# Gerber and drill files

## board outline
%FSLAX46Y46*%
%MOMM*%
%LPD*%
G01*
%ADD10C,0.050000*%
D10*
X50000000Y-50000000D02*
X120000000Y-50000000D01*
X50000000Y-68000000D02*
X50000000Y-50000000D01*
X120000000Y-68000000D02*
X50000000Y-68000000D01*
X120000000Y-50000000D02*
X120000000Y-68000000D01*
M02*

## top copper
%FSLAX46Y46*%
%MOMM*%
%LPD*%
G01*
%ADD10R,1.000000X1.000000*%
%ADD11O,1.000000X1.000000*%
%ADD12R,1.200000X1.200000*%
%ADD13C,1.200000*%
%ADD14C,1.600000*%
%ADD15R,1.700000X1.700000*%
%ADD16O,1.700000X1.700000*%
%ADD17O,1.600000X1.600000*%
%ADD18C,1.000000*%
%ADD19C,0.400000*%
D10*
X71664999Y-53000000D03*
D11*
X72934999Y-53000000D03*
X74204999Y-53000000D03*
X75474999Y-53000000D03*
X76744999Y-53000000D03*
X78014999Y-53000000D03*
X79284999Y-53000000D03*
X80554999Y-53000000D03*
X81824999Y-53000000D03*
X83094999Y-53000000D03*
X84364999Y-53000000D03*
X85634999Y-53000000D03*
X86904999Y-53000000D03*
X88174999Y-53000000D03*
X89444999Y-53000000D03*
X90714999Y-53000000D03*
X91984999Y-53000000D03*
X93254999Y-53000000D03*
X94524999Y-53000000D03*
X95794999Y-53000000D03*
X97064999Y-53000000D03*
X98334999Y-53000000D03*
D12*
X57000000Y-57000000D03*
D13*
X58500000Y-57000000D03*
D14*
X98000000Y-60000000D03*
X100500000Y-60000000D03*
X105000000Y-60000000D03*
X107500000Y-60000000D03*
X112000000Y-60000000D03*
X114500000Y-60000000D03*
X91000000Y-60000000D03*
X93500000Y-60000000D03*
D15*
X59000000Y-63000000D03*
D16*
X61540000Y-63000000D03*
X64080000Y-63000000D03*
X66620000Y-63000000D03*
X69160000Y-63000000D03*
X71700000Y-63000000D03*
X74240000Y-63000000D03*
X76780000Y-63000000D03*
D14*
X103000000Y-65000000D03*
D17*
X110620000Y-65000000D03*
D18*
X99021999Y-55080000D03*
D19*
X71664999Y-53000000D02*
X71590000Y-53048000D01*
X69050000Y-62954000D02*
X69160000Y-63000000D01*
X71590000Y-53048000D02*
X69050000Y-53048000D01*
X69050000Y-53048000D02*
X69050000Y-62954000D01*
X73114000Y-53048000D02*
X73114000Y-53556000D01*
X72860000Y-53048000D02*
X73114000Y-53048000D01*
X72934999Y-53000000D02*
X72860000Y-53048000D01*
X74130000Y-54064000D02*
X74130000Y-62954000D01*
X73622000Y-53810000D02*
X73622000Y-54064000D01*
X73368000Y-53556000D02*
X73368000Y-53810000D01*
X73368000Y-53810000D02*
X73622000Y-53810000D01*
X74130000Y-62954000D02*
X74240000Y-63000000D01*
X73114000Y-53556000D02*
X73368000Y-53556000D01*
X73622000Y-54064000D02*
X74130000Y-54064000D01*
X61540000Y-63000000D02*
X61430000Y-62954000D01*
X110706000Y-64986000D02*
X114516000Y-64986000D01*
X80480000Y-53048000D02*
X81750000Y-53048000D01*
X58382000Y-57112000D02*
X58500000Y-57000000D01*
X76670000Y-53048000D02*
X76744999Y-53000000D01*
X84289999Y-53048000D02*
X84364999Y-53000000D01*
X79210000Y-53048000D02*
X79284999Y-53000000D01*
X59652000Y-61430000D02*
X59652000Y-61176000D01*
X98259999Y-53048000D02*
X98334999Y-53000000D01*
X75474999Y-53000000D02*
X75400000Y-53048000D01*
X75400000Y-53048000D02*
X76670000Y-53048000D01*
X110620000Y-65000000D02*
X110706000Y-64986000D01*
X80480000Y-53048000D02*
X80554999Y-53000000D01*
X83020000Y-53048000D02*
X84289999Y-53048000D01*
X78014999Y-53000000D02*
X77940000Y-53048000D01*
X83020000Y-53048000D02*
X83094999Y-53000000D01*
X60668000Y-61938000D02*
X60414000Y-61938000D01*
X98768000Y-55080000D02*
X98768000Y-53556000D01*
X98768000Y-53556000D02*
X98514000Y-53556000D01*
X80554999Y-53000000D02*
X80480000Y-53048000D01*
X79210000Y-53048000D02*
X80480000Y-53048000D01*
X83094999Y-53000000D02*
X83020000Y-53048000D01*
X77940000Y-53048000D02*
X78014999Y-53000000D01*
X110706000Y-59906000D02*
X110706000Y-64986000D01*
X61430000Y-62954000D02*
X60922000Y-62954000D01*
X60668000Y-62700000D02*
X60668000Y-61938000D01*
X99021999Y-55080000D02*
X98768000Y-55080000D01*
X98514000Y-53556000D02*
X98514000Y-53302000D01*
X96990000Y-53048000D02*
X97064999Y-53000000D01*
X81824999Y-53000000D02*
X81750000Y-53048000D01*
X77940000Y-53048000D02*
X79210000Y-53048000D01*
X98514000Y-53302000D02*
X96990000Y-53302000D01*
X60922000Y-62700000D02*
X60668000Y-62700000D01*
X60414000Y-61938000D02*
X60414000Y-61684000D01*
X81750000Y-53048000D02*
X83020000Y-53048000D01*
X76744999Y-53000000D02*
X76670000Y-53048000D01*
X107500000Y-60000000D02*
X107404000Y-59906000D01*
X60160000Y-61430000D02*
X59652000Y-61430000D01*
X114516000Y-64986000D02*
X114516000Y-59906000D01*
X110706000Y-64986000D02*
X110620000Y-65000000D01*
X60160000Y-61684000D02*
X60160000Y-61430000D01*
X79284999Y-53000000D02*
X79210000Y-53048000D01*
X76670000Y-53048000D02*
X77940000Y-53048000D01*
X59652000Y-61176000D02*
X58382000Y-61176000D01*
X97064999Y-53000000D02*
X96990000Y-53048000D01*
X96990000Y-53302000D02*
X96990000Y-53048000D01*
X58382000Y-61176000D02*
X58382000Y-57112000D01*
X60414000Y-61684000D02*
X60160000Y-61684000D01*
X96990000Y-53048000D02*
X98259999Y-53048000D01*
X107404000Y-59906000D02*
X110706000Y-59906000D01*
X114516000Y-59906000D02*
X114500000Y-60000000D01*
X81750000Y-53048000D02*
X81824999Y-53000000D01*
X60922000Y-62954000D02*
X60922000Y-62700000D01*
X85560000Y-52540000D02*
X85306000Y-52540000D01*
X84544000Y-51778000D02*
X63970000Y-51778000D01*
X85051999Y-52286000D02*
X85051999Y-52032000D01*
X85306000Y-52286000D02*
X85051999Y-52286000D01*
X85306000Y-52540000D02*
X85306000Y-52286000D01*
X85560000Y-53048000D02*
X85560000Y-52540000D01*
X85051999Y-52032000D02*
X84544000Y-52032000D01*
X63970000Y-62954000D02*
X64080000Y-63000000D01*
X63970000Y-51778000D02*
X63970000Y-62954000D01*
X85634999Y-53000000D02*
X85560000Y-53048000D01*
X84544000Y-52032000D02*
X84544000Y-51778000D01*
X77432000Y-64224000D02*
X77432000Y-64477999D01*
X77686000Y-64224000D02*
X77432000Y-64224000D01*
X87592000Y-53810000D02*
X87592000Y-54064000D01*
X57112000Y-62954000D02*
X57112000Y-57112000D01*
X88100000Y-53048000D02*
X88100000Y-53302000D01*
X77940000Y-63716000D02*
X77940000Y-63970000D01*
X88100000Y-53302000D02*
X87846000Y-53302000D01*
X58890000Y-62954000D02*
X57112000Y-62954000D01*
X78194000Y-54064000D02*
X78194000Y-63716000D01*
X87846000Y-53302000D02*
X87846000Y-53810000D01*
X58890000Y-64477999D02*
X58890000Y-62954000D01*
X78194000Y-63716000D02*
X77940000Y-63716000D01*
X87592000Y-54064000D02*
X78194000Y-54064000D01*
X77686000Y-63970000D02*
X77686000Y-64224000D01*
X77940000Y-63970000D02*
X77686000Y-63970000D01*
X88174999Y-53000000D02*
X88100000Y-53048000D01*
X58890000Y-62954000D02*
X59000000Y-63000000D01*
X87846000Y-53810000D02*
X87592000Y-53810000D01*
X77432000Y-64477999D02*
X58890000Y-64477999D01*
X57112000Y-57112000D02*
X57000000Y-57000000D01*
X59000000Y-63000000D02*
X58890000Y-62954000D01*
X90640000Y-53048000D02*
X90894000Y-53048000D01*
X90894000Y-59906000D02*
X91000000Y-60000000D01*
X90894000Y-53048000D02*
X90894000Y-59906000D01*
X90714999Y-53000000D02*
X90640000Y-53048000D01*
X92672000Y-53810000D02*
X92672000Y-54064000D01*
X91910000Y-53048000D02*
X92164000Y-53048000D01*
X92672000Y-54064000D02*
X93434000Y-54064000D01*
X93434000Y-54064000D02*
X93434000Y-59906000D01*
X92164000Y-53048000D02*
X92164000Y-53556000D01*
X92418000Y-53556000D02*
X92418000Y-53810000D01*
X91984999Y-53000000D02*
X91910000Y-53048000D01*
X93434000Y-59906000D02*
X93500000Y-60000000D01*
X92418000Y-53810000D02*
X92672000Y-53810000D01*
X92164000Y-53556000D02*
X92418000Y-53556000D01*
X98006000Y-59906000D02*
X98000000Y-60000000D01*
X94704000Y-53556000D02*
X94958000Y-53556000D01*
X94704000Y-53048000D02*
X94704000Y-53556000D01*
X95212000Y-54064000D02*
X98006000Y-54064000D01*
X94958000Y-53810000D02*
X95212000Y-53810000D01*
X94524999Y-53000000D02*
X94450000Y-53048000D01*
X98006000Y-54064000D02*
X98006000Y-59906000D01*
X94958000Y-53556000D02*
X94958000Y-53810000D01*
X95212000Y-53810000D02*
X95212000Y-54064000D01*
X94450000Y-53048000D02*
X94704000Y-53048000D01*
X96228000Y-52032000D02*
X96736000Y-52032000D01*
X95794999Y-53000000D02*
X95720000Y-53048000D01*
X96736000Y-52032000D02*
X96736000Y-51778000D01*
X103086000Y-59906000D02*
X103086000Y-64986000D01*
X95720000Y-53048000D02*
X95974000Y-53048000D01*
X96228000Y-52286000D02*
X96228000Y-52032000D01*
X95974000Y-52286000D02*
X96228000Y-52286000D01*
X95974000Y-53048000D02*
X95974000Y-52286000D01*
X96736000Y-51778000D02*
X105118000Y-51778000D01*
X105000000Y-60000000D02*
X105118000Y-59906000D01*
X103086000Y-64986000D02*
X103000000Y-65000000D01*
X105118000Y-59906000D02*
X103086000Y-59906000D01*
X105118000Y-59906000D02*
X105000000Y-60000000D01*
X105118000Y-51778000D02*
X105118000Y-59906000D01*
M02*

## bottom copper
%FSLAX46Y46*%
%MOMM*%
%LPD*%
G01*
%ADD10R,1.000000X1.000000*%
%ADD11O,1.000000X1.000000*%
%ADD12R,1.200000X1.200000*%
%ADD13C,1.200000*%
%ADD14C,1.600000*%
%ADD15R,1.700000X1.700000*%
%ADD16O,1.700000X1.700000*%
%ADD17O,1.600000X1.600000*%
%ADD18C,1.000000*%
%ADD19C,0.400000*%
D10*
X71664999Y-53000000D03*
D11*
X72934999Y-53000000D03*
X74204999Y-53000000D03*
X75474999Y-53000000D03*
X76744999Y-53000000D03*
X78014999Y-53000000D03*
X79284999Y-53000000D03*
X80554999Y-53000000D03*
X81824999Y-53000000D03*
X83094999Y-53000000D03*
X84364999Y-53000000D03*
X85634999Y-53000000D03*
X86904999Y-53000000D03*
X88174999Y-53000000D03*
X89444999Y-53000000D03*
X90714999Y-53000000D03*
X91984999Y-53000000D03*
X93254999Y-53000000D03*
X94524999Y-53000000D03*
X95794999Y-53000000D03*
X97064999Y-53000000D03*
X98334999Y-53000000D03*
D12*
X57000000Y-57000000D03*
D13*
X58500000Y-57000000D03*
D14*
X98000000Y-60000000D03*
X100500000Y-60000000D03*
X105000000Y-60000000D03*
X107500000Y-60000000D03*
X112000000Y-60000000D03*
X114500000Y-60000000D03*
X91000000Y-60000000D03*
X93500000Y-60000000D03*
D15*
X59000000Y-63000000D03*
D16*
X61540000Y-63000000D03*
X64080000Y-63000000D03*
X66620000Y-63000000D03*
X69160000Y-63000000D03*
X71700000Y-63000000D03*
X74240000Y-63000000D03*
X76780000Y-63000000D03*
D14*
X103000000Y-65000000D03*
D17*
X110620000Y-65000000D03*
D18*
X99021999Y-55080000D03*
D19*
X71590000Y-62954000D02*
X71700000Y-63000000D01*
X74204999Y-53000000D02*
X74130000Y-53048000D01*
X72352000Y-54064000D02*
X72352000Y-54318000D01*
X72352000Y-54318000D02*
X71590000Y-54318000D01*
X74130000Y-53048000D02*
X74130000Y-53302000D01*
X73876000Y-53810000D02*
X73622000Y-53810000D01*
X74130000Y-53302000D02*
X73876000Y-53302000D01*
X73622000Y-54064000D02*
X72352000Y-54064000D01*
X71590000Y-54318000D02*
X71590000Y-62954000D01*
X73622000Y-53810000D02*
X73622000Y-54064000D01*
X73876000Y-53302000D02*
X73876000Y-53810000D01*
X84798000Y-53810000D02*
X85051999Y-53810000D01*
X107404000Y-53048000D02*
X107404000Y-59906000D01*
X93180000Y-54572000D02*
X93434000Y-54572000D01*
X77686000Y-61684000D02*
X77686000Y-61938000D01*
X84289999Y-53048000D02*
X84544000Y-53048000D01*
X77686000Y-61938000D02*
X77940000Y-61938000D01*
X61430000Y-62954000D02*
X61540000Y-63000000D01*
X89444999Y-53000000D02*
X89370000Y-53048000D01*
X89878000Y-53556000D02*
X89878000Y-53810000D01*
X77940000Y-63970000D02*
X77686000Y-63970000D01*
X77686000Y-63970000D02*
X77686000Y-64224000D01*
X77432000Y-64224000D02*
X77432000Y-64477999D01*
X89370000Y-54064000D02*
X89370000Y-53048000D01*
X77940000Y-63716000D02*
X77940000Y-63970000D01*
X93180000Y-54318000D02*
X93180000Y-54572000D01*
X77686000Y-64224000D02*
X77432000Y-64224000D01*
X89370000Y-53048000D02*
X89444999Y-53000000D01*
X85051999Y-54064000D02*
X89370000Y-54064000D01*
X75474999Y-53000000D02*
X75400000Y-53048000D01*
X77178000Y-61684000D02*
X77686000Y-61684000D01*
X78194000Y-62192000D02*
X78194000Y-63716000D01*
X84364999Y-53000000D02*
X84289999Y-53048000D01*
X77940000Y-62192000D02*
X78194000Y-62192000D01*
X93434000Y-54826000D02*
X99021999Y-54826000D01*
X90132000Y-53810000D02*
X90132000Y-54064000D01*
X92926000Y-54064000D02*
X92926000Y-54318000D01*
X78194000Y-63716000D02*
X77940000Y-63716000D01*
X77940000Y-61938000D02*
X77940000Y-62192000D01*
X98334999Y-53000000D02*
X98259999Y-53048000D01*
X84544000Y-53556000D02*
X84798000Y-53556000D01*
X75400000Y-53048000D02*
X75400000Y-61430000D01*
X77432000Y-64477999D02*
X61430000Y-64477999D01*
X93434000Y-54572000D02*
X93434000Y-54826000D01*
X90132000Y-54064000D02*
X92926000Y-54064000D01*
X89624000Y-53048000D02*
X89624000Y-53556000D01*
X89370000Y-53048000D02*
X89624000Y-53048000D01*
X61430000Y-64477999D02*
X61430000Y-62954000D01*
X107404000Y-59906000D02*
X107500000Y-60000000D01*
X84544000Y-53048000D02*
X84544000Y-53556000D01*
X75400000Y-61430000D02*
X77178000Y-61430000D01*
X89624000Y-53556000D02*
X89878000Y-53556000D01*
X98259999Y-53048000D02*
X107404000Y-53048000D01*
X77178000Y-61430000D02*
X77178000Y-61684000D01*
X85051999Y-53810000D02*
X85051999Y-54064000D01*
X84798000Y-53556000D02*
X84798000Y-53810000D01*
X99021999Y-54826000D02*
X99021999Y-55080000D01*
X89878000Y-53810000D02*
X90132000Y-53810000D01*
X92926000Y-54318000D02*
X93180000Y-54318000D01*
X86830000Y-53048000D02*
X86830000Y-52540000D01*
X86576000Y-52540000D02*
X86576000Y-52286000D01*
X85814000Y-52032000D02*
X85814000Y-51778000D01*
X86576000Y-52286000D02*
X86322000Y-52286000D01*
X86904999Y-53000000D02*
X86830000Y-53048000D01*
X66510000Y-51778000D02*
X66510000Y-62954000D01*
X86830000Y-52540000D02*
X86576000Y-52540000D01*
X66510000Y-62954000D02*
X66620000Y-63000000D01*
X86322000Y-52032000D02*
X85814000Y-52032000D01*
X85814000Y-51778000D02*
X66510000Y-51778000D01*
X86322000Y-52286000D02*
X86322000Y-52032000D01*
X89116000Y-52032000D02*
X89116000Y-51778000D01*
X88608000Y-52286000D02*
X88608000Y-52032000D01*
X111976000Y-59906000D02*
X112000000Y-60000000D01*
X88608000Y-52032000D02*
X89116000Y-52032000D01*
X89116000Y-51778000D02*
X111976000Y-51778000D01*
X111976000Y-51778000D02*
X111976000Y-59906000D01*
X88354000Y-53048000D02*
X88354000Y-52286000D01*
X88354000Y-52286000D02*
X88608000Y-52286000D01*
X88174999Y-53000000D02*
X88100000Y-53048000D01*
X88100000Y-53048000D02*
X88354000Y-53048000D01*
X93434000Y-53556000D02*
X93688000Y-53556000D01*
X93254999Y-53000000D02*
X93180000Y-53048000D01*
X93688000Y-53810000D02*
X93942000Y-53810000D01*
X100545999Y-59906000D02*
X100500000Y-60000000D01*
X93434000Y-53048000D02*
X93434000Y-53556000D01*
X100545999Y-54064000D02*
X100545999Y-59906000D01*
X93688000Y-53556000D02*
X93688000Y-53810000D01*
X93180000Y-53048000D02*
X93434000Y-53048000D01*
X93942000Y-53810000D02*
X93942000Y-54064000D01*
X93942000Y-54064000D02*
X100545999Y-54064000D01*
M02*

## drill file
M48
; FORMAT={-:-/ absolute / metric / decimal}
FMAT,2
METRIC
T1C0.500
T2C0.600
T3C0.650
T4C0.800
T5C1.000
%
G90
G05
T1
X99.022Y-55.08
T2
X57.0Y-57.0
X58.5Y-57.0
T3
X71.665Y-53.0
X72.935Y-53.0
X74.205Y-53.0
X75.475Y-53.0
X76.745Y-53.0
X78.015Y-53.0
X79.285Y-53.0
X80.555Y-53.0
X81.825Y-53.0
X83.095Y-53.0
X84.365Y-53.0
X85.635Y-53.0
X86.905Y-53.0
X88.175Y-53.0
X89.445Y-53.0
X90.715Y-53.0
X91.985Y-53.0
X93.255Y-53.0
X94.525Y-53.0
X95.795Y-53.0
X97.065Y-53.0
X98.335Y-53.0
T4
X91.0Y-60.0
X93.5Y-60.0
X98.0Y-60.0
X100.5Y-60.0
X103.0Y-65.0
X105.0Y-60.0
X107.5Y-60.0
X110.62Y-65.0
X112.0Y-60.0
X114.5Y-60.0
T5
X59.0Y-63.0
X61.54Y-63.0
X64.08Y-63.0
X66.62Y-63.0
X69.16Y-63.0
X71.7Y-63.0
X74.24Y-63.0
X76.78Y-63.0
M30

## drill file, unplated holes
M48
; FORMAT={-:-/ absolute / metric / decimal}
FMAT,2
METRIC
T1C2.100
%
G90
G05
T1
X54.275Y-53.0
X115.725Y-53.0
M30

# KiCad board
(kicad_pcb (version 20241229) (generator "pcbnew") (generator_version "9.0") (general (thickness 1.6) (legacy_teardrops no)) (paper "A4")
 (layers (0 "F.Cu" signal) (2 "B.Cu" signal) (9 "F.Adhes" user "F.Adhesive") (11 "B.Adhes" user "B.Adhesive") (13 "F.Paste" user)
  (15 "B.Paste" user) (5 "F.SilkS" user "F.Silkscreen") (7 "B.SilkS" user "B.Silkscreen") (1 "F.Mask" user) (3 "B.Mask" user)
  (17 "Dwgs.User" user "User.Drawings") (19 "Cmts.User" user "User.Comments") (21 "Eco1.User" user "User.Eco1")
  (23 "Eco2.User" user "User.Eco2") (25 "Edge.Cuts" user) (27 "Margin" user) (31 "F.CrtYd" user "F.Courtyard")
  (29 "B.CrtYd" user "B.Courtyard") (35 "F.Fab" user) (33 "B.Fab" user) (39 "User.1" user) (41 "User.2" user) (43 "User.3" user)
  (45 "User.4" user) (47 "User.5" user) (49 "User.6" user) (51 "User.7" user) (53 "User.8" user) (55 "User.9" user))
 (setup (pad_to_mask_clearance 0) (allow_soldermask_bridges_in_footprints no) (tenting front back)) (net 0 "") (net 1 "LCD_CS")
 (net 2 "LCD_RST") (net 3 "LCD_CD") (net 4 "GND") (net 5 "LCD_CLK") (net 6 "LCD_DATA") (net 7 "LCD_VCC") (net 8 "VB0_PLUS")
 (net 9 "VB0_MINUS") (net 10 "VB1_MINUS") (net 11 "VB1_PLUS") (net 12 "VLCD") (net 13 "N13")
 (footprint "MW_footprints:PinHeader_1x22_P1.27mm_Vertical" (layer "F.Cu") (at 71.664999 53 90)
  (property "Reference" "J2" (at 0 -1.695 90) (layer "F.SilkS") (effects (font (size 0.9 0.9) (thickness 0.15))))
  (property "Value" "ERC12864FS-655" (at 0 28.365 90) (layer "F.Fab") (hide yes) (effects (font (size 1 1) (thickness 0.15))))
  (pad "1" thru_hole rect (at 0 0 90) (size 1 1) (drill 0.65) (layers "*.Cu" "*.Mask") (remove_unused_layers no) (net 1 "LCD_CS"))
  (pad "2" thru_hole oval (at 0 1.27 90) (size 1 1) (drill 0.65) (layers "*.Cu" "*.Mask") (remove_unused_layers no) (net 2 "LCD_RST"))
  (pad "3" thru_hole oval (at 0 2.54 90) (size 1 1) (drill 0.65) (layers "*.Cu" "*.Mask") (remove_unused_layers no) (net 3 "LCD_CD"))
  (pad "4" thru_hole oval (at 0 3.81 90) (size 1 1) (drill 0.65) (layers "*.Cu" "*.Mask") (remove_unused_layers no) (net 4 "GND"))
  (pad "5" thru_hole oval (at 0 5.08 90) (size 1 1) (drill 0.65) (layers "*.Cu" "*.Mask") (remove_unused_layers no) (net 4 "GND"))
  (pad "6" thru_hole oval (at 0 6.35 90) (size 1 1) (drill 0.65) (layers "*.Cu" "*.Mask") (remove_unused_layers no) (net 4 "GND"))
  (pad "7" thru_hole oval (at 0 7.62 90) (size 1 1) (drill 0.65) (layers "*.Cu" "*.Mask") (remove_unused_layers no) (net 4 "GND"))
  (pad "8" thru_hole oval (at 0 8.89 90) (size 1 1) (drill 0.65) (layers "*.Cu" "*.Mask") (remove_unused_layers no) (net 4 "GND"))
  (pad "9" thru_hole oval (at 0 10.16 90) (size 1 1) (drill 0.65) (layers "*.Cu" "*.Mask") (remove_unused_layers no) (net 4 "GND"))
  (pad "10" thru_hole oval (at 0 11.43 90) (size 1 1) (drill 0.65) (layers "*.Cu" "*.Mask") (remove_unused_layers no) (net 4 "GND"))
  (pad "11" thru_hole oval (at 0 12.7 90) (size 1 1) (drill 0.65) (layers "*.Cu" "*.Mask") (remove_unused_layers no) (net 4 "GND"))
  (pad "12" thru_hole oval (at 0 13.97 90) (size 1 1) (drill 0.65) (layers "*.Cu" "*.Mask") (remove_unused_layers no) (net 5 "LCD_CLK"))
  (pad "13" thru_hole oval (at 0 15.24 90) (size 1 1) (drill 0.65) (layers "*.Cu" "*.Mask") (remove_unused_layers no) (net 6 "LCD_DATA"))
  (pad "14" thru_hole oval (at 0 16.51 90) (size 1 1) (drill 0.65) (layers "*.Cu" "*.Mask") (remove_unused_layers no) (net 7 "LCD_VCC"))
  (pad "15" thru_hole oval (at 0 17.78 90) (size 1 1) (drill 0.65) (layers "*.Cu" "*.Mask") (remove_unused_layers no) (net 4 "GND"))
  (pad "16" thru_hole oval (at 0 19.05 90) (size 1 1) (drill 0.65) (layers "*.Cu" "*.Mask") (remove_unused_layers no) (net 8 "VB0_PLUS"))
  (pad "17" thru_hole oval (at 0 20.32 90) (size 1 1) (drill 0.65) (layers "*.Cu" "*.Mask") (remove_unused_layers no) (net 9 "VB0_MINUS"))
  (pad "18" thru_hole oval (at 0 21.59 90) (size 1 1) (drill 0.65) (layers "*.Cu" "*.Mask") (remove_unused_layers no) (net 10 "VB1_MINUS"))
  (pad "19" thru_hole oval (at 0 22.86 90) (size 1 1) (drill 0.65) (layers "*.Cu" "*.Mask") (remove_unused_layers no) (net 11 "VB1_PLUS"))
  (pad "20" thru_hole oval (at 0 24.13 90) (size 1 1) (drill 0.65) (layers "*.Cu" "*.Mask") (remove_unused_layers no) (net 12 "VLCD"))
  (pad "21" thru_hole oval (at 0 25.4 90) (size 1 1) (drill 0.65) (layers "*.Cu" "*.Mask") (remove_unused_layers no) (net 4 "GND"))
  (pad "22" thru_hole oval (at 0 26.67 90) (size 1 1) (drill 0.65) (layers "*.Cu" "*.Mask") (remove_unused_layers no) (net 4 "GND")))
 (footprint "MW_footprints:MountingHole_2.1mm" (layer "F.Cu") (at 54.275 53)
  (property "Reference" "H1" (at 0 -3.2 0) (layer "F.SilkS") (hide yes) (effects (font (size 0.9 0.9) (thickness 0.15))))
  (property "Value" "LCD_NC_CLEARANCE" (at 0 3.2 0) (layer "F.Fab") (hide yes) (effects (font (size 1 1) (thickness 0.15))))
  (pad "" np_thru_hole circle (at 0 0) (size 2.1 2.1) (drill 2.1) (layers "*.Cu" "*.Mask")))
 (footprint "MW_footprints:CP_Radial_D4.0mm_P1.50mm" (layer "F.Cu") (at 57 57)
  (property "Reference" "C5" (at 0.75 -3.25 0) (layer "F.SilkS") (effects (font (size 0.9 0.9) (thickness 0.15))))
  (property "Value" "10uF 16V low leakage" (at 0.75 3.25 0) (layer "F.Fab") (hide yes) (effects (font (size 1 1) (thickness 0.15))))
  (pad "1" thru_hole rect (at 0 0) (size 1.2 1.2) (drill 0.6) (layers "*.Cu" "*.Mask") (remove_unused_layers no) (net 7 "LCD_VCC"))
  (pad "2" thru_hole circle (at 1.5 0) (size 1.2 1.2) (drill 0.6) (layers "*.Cu" "*.Mask") (remove_unused_layers no) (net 4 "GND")))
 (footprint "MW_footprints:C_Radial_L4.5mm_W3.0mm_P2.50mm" (layer "F.Cu") (at 98 60)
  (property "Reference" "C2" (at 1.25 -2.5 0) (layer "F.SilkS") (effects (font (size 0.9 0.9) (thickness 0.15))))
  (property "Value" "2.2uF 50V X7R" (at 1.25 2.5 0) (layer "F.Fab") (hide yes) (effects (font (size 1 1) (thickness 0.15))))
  (pad "1" thru_hole circle (at 0 0) (size 1.6 1.6) (drill 0.8) (layers "*.Cu" "*.Mask") (remove_unused_layers no) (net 11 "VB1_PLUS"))
  (pad "2" thru_hole circle (at 2.5 0) (size 1.6 1.6) (drill 0.8) (layers "*.Cu" "*.Mask") (remove_unused_layers no) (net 10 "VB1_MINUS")))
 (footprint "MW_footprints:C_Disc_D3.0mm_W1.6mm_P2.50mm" (layer "F.Cu") (at 105 60)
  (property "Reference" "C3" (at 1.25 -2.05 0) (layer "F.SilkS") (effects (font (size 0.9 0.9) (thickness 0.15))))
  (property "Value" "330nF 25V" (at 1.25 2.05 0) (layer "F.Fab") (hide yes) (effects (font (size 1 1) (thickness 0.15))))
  (pad "1" thru_hole circle (at 0 0) (size 1.6 1.6) (drill 0.8) (layers "*.Cu" "*.Mask") (remove_unused_layers no) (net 12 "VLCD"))
  (pad "2" thru_hole circle (at 2.5 0) (size 1.6 1.6) (drill 0.8) (layers "*.Cu" "*.Mask") (remove_unused_layers no) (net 4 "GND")))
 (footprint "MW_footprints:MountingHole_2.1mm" (layer "F.Cu") (at 115.725 53)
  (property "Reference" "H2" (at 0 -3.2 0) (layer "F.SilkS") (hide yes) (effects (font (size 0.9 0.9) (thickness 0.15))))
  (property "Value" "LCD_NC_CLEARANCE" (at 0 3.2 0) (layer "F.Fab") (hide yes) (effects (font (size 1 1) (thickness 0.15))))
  (pad "" np_thru_hole circle (at 0 0) (size 2.1 2.1) (drill 2.1) (layers "*.Cu" "*.Mask")))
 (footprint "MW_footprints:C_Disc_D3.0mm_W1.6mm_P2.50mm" (layer "F.Cu") (at 112 60)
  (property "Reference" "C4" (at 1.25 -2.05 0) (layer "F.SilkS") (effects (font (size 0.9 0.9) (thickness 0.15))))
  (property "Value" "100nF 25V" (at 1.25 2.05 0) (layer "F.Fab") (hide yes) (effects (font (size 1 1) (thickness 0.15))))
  (pad "1" thru_hole circle (at 0 0) (size 1.6 1.6) (drill 0.8) (layers "*.Cu" "*.Mask") (remove_unused_layers no) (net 7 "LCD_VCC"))
  (pad "2" thru_hole circle (at 2.5 0) (size 1.6 1.6) (drill 0.8) (layers "*.Cu" "*.Mask") (remove_unused_layers no) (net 4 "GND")))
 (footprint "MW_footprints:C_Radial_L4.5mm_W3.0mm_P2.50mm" (layer "F.Cu") (at 91 60)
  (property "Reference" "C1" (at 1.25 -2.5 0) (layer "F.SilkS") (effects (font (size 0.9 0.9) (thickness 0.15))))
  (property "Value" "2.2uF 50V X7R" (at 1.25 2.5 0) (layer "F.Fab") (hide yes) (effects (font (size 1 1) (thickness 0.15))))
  (pad "1" thru_hole circle (at 0 0) (size 1.6 1.6) (drill 0.8) (layers "*.Cu" "*.Mask") (remove_unused_layers no) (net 8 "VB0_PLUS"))
  (pad "2" thru_hole circle (at 2.5 0) (size 1.6 1.6) (drill 0.8) (layers "*.Cu" "*.Mask") (remove_unused_layers no) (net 9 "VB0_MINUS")))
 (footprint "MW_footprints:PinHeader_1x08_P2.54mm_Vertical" (layer "F.Cu") (at 59 63 90)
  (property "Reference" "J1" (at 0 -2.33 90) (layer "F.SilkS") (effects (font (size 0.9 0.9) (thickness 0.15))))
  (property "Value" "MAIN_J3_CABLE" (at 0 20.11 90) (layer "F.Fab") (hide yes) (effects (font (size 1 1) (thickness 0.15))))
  (pad "1" thru_hole rect (at 0 0 90) (size 1.7 1.7) (drill 1) (layers "*.Cu" "*.Mask") (remove_unused_layers no) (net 7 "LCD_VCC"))
  (pad "2" thru_hole oval (at 0 2.54 90) (size 1.7 1.7) (drill 1) (layers "*.Cu" "*.Mask") (remove_unused_layers no) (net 4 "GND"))
  (pad "3" thru_hole oval (at 0 5.08 90) (size 1.7 1.7) (drill 1) (layers "*.Cu" "*.Mask") (remove_unused_layers no) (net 5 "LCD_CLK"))
  (pad "4" thru_hole oval (at 0 7.62 90) (size 1.7 1.7) (drill 1) (layers "*.Cu" "*.Mask") (remove_unused_layers no) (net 6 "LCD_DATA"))
  (pad "5" thru_hole oval (at 0 10.16 90) (size 1.7 1.7) (drill 1) (layers "*.Cu" "*.Mask") (remove_unused_layers no) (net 1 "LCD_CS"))
  (pad "6" thru_hole oval (at 0 12.7 90) (size 1.7 1.7) (drill 1) (layers "*.Cu" "*.Mask") (remove_unused_layers no) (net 3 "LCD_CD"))
  (pad "7" thru_hole oval (at 0 15.24 90) (size 1.7 1.7) (drill 1) (layers "*.Cu" "*.Mask") (remove_unused_layers no) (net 2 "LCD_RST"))
  (pad "8" thru_hole oval (at 0 17.78 90) (size 1.7 1.7) (drill 1) (layers "*.Cu" "*.Mask") (remove_unused_layers no) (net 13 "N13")))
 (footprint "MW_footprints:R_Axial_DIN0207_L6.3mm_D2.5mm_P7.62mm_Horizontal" (layer "F.Cu") (at 103 65)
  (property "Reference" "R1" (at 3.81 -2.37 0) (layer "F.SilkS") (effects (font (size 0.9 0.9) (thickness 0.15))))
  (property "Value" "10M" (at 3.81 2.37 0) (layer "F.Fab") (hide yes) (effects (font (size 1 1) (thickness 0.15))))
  (pad "1" thru_hole circle (at 0 0) (size 1.6 1.6) (drill 0.8) (layers "*.Cu" "*.Mask") (remove_unused_layers no) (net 12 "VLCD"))
  (pad "2" thru_hole oval (at 7.62 0) (size 1.6 1.6) (drill 0.8) (layers "*.Cu" "*.Mask") (remove_unused_layers no) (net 4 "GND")))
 (gr_line (start 50 50) (end 120 50) (stroke (width 0.05) (type default)) (layer "Edge.Cuts"))
 (gr_line (start 50 68) (end 50 50) (stroke (width 0.05) (type default)) (layer "Edge.Cuts"))
 (gr_line (start 120 68) (end 50 68) (stroke (width 0.05) (type default)) (layer "Edge.Cuts"))
 (gr_line (start 120 50) (end 120 68) (stroke (width 0.05) (type default)) (layer "Edge.Cuts"))
 (segment (start 71.664999 53) (end 71.59 53.048) (width 0.4) (layer "F.Cu") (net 1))
 (segment (start 69.05 62.954) (end 69.16 63) (width 0.4) (layer "F.Cu") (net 1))
 (segment (start 71.59 53.048) (end 69.05 53.048) (width 0.4) (layer "F.Cu") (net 1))
 (segment (start 69.05 53.048) (end 69.05 62.954) (width 0.4) (layer "F.Cu") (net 1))
 (segment (start 73.114 53.048) (end 73.114 53.556) (width 0.4) (layer "F.Cu") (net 2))
 (segment (start 72.86 53.048) (end 73.114 53.048) (width 0.4) (layer "F.Cu") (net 2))
 (segment (start 72.934999 53) (end 72.86 53.048) (width 0.4) (layer "F.Cu") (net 2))
 (segment (start 74.13 54.064) (end 74.13 62.954) (width 0.4) (layer "F.Cu") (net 2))
 (segment (start 73.622 53.81) (end 73.622 54.064) (width 0.4) (layer "F.Cu") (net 2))
 (segment (start 73.368 53.556) (end 73.368 53.81) (width 0.4) (layer "F.Cu") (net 2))
 (segment (start 73.368 53.81) (end 73.622 53.81) (width 0.4) (layer "F.Cu") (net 2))
 (segment (start 74.13 62.954) (end 74.24 63) (width 0.4) (layer "F.Cu") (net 2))
 (segment (start 73.114 53.556) (end 73.368 53.556) (width 0.4) (layer "F.Cu") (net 2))
 (segment (start 73.622 54.064) (end 74.13 54.064) (width 0.4) (layer "F.Cu") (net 2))
 (segment (start 71.59 62.954) (end 71.7 63) (width 0.4) (layer "B.Cu") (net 3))
 (segment (start 74.204999 53) (end 74.13 53.048) (width 0.4) (layer "B.Cu") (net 3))
 (segment (start 72.352 54.064) (end 72.352 54.318) (width 0.4) (layer "B.Cu") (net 3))
 (segment (start 72.352 54.318) (end 71.59 54.318) (width 0.4) (layer "B.Cu") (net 3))
 (segment (start 74.13 53.048) (end 74.13 53.302) (width 0.4) (layer "B.Cu") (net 3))
 (segment (start 73.876 53.81) (end 73.622 53.81) (width 0.4) (layer "B.Cu") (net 3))
 (segment (start 74.13 53.302) (end 73.876 53.302) (width 0.4) (layer "B.Cu") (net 3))
 (segment (start 73.622 54.064) (end 72.352 54.064) (width 0.4) (layer "B.Cu") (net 3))
 (segment (start 71.59 54.318) (end 71.59 62.954) (width 0.4) (layer "B.Cu") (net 3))
 (segment (start 73.622 53.81) (end 73.622 54.064) (width 0.4) (layer "B.Cu") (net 3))
 (segment (start 73.876 53.302) (end 73.876 53.81) (width 0.4) (layer "B.Cu") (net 3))
 (segment (start 61.54 63) (end 61.43 62.954) (width 0.4) (layer "F.Cu") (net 4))
 (segment (start 110.706 64.986) (end 114.516 64.986) (width 0.4) (layer "F.Cu") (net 4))
 (segment (start 80.48 53.048) (end 81.75 53.048) (width 0.4) (layer "F.Cu") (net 4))
 (segment (start 58.382 57.112) (end 58.5 57) (width 0.4) (layer "F.Cu") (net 4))
 (segment (start 76.67 53.048) (end 76.744999 53) (width 0.4) (layer "F.Cu") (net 4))
 (segment (start 84.289999 53.048) (end 84.364999 53) (width 0.4) (layer "F.Cu") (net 4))
 (segment (start 79.21 53.048) (end 79.284999 53) (width 0.4) (layer "F.Cu") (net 4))
 (segment (start 59.652 61.43) (end 59.652 61.176) (width 0.4) (layer "F.Cu") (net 4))
 (segment (start 98.259999 53.048) (end 98.334999 53) (width 0.4) (layer "F.Cu") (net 4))
 (segment (start 75.474999 53) (end 75.4 53.048) (width 0.4) (layer "F.Cu") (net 4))
 (segment (start 75.4 53.048) (end 76.67 53.048) (width 0.4) (layer "F.Cu") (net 4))
 (segment (start 110.62 65) (end 110.706 64.986) (width 0.4) (layer "F.Cu") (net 4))
 (segment (start 80.48 53.048) (end 80.554999 53) (width 0.4) (layer "F.Cu") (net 4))
 (segment (start 83.02 53.048) (end 84.289999 53.048) (width 0.4) (layer "F.Cu") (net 4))
 (segment (start 78.014999 53) (end 77.94 53.048) (width 0.4) (layer "F.Cu") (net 4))
 (segment (start 83.02 53.048) (end 83.094999 53) (width 0.4) (layer "F.Cu") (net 4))
 (segment (start 60.668 61.938) (end 60.414 61.938) (width 0.4) (layer "F.Cu") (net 4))
 (segment (start 98.768 55.08) (end 98.768 53.556) (width 0.4) (layer "F.Cu") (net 4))
 (segment (start 98.768 53.556) (end 98.514 53.556) (width 0.4) (layer "F.Cu") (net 4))
 (segment (start 80.554999 53) (end 80.48 53.048) (width 0.4) (layer "F.Cu") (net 4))
 (segment (start 79.21 53.048) (end 80.48 53.048) (width 0.4) (layer "F.Cu") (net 4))
 (segment (start 83.094999 53) (end 83.02 53.048) (width 0.4) (layer "F.Cu") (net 4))
 (segment (start 77.94 53.048) (end 78.014999 53) (width 0.4) (layer "F.Cu") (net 4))
 (segment (start 110.706 59.906) (end 110.706 64.986) (width 0.4) (layer "F.Cu") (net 4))
 (segment (start 61.43 62.954) (end 60.922 62.954) (width 0.4) (layer "F.Cu") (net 4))
 (segment (start 60.668 62.7) (end 60.668 61.938) (width 0.4) (layer "F.Cu") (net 4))
 (segment (start 99.021999 55.08) (end 98.768 55.08) (width 0.4) (layer "F.Cu") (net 4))
 (segment (start 98.514 53.556) (end 98.514 53.302) (width 0.4) (layer "F.Cu") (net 4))
 (segment (start 96.99 53.048) (end 97.064999 53) (width 0.4) (layer "F.Cu") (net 4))
 (segment (start 81.824999 53) (end 81.75 53.048) (width 0.4) (layer "F.Cu") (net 4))
 (segment (start 77.94 53.048) (end 79.21 53.048) (width 0.4) (layer "F.Cu") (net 4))
 (segment (start 98.514 53.302) (end 96.99 53.302) (width 0.4) (layer "F.Cu") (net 4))
 (segment (start 60.922 62.7) (end 60.668 62.7) (width 0.4) (layer "F.Cu") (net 4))
 (segment (start 60.414 61.938) (end 60.414 61.684) (width 0.4) (layer "F.Cu") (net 4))
 (segment (start 81.75 53.048) (end 83.02 53.048) (width 0.4) (layer "F.Cu") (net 4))
 (segment (start 76.744999 53) (end 76.67 53.048) (width 0.4) (layer "F.Cu") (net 4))
 (segment (start 107.5 60) (end 107.404 59.906) (width 0.4) (layer "F.Cu") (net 4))
 (segment (start 60.16 61.43) (end 59.652 61.43) (width 0.4) (layer "F.Cu") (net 4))
 (segment (start 114.516 64.986) (end 114.516 59.906) (width 0.4) (layer "F.Cu") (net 4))
 (segment (start 110.706 64.986) (end 110.62 65) (width 0.4) (layer "F.Cu") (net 4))
 (segment (start 60.16 61.684) (end 60.16 61.43) (width 0.4) (layer "F.Cu") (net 4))
 (segment (start 79.284999 53) (end 79.21 53.048) (width 0.4) (layer "F.Cu") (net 4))
 (segment (start 76.67 53.048) (end 77.94 53.048) (width 0.4) (layer "F.Cu") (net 4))
 (segment (start 59.652 61.176) (end 58.382 61.176) (width 0.4) (layer "F.Cu") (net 4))
 (segment (start 97.064999 53) (end 96.99 53.048) (width 0.4) (layer "F.Cu") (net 4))
 (segment (start 96.99 53.302) (end 96.99 53.048) (width 0.4) (layer "F.Cu") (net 4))
 (segment (start 58.382 61.176) (end 58.382 57.112) (width 0.4) (layer "F.Cu") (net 4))
 (segment (start 60.414 61.684) (end 60.16 61.684) (width 0.4) (layer "F.Cu") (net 4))
 (segment (start 96.99 53.048) (end 98.259999 53.048) (width 0.4) (layer "F.Cu") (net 4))
 (segment (start 107.404 59.906) (end 110.706 59.906) (width 0.4) (layer "F.Cu") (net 4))
 (segment (start 114.516 59.906) (end 114.5 60) (width 0.4) (layer "F.Cu") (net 4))
 (segment (start 81.75 53.048) (end 81.824999 53) (width 0.4) (layer "F.Cu") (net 4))
 (segment (start 60.922 62.954) (end 60.922 62.7) (width 0.4) (layer "F.Cu") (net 4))
 (via (at 99.021999 55.08) (size 1) (drill 0.5) (layers "F.Cu" "B.Cu") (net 4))
 (segment (start 84.798 53.81) (end 85.051999 53.81) (width 0.4) (layer "B.Cu") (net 4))
 (segment (start 107.404 53.048) (end 107.404 59.906) (width 0.4) (layer "B.Cu") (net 4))
 (segment (start 93.18 54.572) (end 93.434 54.572) (width 0.4) (layer "B.Cu") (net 4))
 (segment (start 77.686 61.684) (end 77.686 61.938) (width 0.4) (layer "B.Cu") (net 4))
 (segment (start 84.289999 53.048) (end 84.544 53.048) (width 0.4) (layer "B.Cu") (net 4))
 (segment (start 77.686 61.938) (end 77.94 61.938) (width 0.4) (layer "B.Cu") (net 4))
 (segment (start 61.43 62.954) (end 61.54 63) (width 0.4) (layer "B.Cu") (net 4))
 (segment (start 89.444999 53) (end 89.37 53.048) (width 0.4) (layer "B.Cu") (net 4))
 (segment (start 89.878 53.556) (end 89.878 53.81) (width 0.4) (layer "B.Cu") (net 4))
 (segment (start 77.94 63.97) (end 77.686 63.97) (width 0.4) (layer "B.Cu") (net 4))
 (segment (start 77.686 63.97) (end 77.686 64.224) (width 0.4) (layer "B.Cu") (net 4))
 (segment (start 77.432 64.224) (end 77.432 64.477999) (width 0.4) (layer "B.Cu") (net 4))
 (segment (start 89.37 54.064) (end 89.37 53.048) (width 0.4) (layer "B.Cu") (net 4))
 (segment (start 77.94 63.716) (end 77.94 63.97) (width 0.4) (layer "B.Cu") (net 4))
 (segment (start 93.18 54.318) (end 93.18 54.572) (width 0.4) (layer "B.Cu") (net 4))
 (segment (start 77.686 64.224) (end 77.432 64.224) (width 0.4) (layer "B.Cu") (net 4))
 (segment (start 89.37 53.048) (end 89.444999 53) (width 0.4) (layer "B.Cu") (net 4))
 (segment (start 85.051999 54.064) (end 89.37 54.064) (width 0.4) (layer "B.Cu") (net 4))
 (segment (start 75.474999 53) (end 75.4 53.048) (width 0.4) (layer "B.Cu") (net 4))
 (segment (start 77.178 61.684) (end 77.686 61.684) (width 0.4) (layer "B.Cu") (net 4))
 (segment (start 78.194 62.192) (end 78.194 63.716) (width 0.4) (layer "B.Cu") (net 4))
 (segment (start 84.364999 53) (end 84.289999 53.048) (width 0.4) (layer "B.Cu") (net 4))
 (segment (start 77.94 62.192) (end 78.194 62.192) (width 0.4) (layer "B.Cu") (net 4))
 (segment (start 93.434 54.826) (end 99.021999 54.826) (width 0.4) (layer "B.Cu") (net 4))
 (segment (start 90.132 53.81) (end 90.132 54.064) (width 0.4) (layer "B.Cu") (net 4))
 (segment (start 92.926 54.064) (end 92.926 54.318) (width 0.4) (layer "B.Cu") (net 4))
 (segment (start 78.194 63.716) (end 77.94 63.716) (width 0.4) (layer "B.Cu") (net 4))
 (segment (start 77.94 61.938) (end 77.94 62.192) (width 0.4) (layer "B.Cu") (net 4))
 (segment (start 98.334999 53) (end 98.259999 53.048) (width 0.4) (layer "B.Cu") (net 4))
 (segment (start 84.544 53.556) (end 84.798 53.556) (width 0.4) (layer "B.Cu") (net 4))
 (segment (start 75.4 53.048) (end 75.4 61.43) (width 0.4) (layer "B.Cu") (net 4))
 (segment (start 77.432 64.477999) (end 61.43 64.477999) (width 0.4) (layer "B.Cu") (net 4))
 (segment (start 93.434 54.572) (end 93.434 54.826) (width 0.4) (layer "B.Cu") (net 4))
 (segment (start 90.132 54.064) (end 92.926 54.064) (width 0.4) (layer "B.Cu") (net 4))
 (segment (start 89.624 53.048) (end 89.624 53.556) (width 0.4) (layer "B.Cu") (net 4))
 (segment (start 89.37 53.048) (end 89.624 53.048) (width 0.4) (layer "B.Cu") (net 4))
 (segment (start 61.43 64.477999) (end 61.43 62.954) (width 0.4) (layer "B.Cu") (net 4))
 (segment (start 107.404 59.906) (end 107.5 60) (width 0.4) (layer "B.Cu") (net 4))
 (segment (start 84.544 53.048) (end 84.544 53.556) (width 0.4) (layer "B.Cu") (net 4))
 (segment (start 75.4 61.43) (end 77.178 61.43) (width 0.4) (layer "B.Cu") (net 4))
 (segment (start 89.624 53.556) (end 89.878 53.556) (width 0.4) (layer "B.Cu") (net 4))
 (segment (start 98.259999 53.048) (end 107.404 53.048) (width 0.4) (layer "B.Cu") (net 4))
 (segment (start 77.178 61.43) (end 77.178 61.684) (width 0.4) (layer "B.Cu") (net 4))
 (segment (start 85.051999 53.81) (end 85.051999 54.064) (width 0.4) (layer "B.Cu") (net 4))
 (segment (start 84.798 53.556) (end 84.798 53.81) (width 0.4) (layer "B.Cu") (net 4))
 (segment (start 99.021999 54.826) (end 99.021999 55.08) (width 0.4) (layer "B.Cu") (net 4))
 (segment (start 89.878 53.81) (end 90.132 53.81) (width 0.4) (layer "B.Cu") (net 4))
 (segment (start 92.926 54.318) (end 93.18 54.318) (width 0.4) (layer "B.Cu") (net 4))
 (segment (start 85.56 52.54) (end 85.306 52.54) (width 0.4) (layer "F.Cu") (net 5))
 (segment (start 84.544 51.778) (end 63.97 51.778) (width 0.4) (layer "F.Cu") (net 5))
 (segment (start 85.051999 52.286) (end 85.051999 52.032) (width 0.4) (layer "F.Cu") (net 5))
 (segment (start 85.306 52.286) (end 85.051999 52.286) (width 0.4) (layer "F.Cu") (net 5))
 (segment (start 85.306 52.54) (end 85.306 52.286) (width 0.4) (layer "F.Cu") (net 5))
 (segment (start 85.56 53.048) (end 85.56 52.54) (width 0.4) (layer "F.Cu") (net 5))
 (segment (start 85.051999 52.032) (end 84.544 52.032) (width 0.4) (layer "F.Cu") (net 5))
 (segment (start 63.97 62.954) (end 64.08 63) (width 0.4) (layer "F.Cu") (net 5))
 (segment (start 63.97 51.778) (end 63.97 62.954) (width 0.4) (layer "F.Cu") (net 5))
 (segment (start 85.634999 53) (end 85.56 53.048) (width 0.4) (layer "F.Cu") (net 5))
 (segment (start 84.544 52.032) (end 84.544 51.778) (width 0.4) (layer "F.Cu") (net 5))
 (segment (start 86.83 53.048) (end 86.83 52.54) (width 0.4) (layer "B.Cu") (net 6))
 (segment (start 86.576 52.54) (end 86.576 52.286) (width 0.4) (layer "B.Cu") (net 6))
 (segment (start 85.814 52.032) (end 85.814 51.778) (width 0.4) (layer "B.Cu") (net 6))
 (segment (start 86.576 52.286) (end 86.322 52.286) (width 0.4) (layer "B.Cu") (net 6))
 (segment (start 86.904999 53) (end 86.83 53.048) (width 0.4) (layer "B.Cu") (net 6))
 (segment (start 66.51 51.778) (end 66.51 62.954) (width 0.4) (layer "B.Cu") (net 6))
 (segment (start 86.83 52.54) (end 86.576 52.54) (width 0.4) (layer "B.Cu") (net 6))
 (segment (start 66.51 62.954) (end 66.62 63) (width 0.4) (layer "B.Cu") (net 6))
 (segment (start 86.322 52.032) (end 85.814 52.032) (width 0.4) (layer "B.Cu") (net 6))
 (segment (start 85.814 51.778) (end 66.51 51.778) (width 0.4) (layer "B.Cu") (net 6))
 (segment (start 86.322 52.286) (end 86.322 52.032) (width 0.4) (layer "B.Cu") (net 6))
 (segment (start 77.432 64.224) (end 77.432 64.477999) (width 0.4) (layer "F.Cu") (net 7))
 (segment (start 77.686 64.224) (end 77.432 64.224) (width 0.4) (layer "F.Cu") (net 7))
 (segment (start 87.592 53.81) (end 87.592 54.064) (width 0.4) (layer "F.Cu") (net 7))
 (segment (start 57.112 62.954) (end 57.112 57.112) (width 0.4) (layer "F.Cu") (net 7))
 (segment (start 88.1 53.048) (end 88.1 53.302) (width 0.4) (layer "F.Cu") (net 7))
 (segment (start 77.94 63.716) (end 77.94 63.97) (width 0.4) (layer "F.Cu") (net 7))
 (segment (start 88.1 53.302) (end 87.846 53.302) (width 0.4) (layer "F.Cu") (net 7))
 (segment (start 58.89 62.954) (end 57.112 62.954) (width 0.4) (layer "F.Cu") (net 7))
 (segment (start 78.194 54.064) (end 78.194 63.716) (width 0.4) (layer "F.Cu") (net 7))
 (segment (start 87.846 53.302) (end 87.846 53.81) (width 0.4) (layer "F.Cu") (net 7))
 (segment (start 58.89 64.477999) (end 58.89 62.954) (width 0.4) (layer "F.Cu") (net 7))
 (segment (start 78.194 63.716) (end 77.94 63.716) (width 0.4) (layer "F.Cu") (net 7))
 (segment (start 87.592 54.064) (end 78.194 54.064) (width 0.4) (layer "F.Cu") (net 7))
 (segment (start 77.686 63.97) (end 77.686 64.224) (width 0.4) (layer "F.Cu") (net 7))
 (segment (start 77.94 63.97) (end 77.686 63.97) (width 0.4) (layer "F.Cu") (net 7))
 (segment (start 88.174999 53) (end 88.1 53.048) (width 0.4) (layer "F.Cu") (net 7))
 (segment (start 58.89 62.954) (end 59 63) (width 0.4) (layer "F.Cu") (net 7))
 (segment (start 87.846 53.81) (end 87.592 53.81) (width 0.4) (layer "F.Cu") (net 7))
 (segment (start 77.432 64.477999) (end 58.89 64.477999) (width 0.4) (layer "F.Cu") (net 7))
 (segment (start 57.112 57.112) (end 57 57) (width 0.4) (layer "F.Cu") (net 7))
 (segment (start 59 63) (end 58.89 62.954) (width 0.4) (layer "F.Cu") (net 7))
 (segment (start 89.116 52.032) (end 89.116 51.778) (width 0.4) (layer "B.Cu") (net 7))
 (segment (start 88.608 52.286) (end 88.608 52.032) (width 0.4) (layer "B.Cu") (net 7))
 (segment (start 111.976 59.906) (end 112 60) (width 0.4) (layer "B.Cu") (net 7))
 (segment (start 88.608 52.032) (end 89.116 52.032) (width 0.4) (layer "B.Cu") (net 7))
 (segment (start 89.116 51.778) (end 111.976 51.778) (width 0.4) (layer "B.Cu") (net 7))
 (segment (start 111.976 51.778) (end 111.976 59.906) (width 0.4) (layer "B.Cu") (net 7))
 (segment (start 88.354 53.048) (end 88.354 52.286) (width 0.4) (layer "B.Cu") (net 7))
 (segment (start 88.354 52.286) (end 88.608 52.286) (width 0.4) (layer "B.Cu") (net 7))
 (segment (start 88.174999 53) (end 88.1 53.048) (width 0.4) (layer "B.Cu") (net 7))
 (segment (start 88.1 53.048) (end 88.354 53.048) (width 0.4) (layer "B.Cu") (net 7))
 (segment (start 90.64 53.048) (end 90.894 53.048) (width 0.4) (layer "F.Cu") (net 8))
 (segment (start 90.894 59.906) (end 91 60) (width 0.4) (layer "F.Cu") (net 8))
 (segment (start 90.894 53.048) (end 90.894 59.906) (width 0.4) (layer "F.Cu") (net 8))
 (segment (start 90.714999 53) (end 90.64 53.048) (width 0.4) (layer "F.Cu") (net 8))
 (segment (start 92.672 53.81) (end 92.672 54.064) (width 0.4) (layer "F.Cu") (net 9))
 (segment (start 91.91 53.048) (end 92.164 53.048) (width 0.4) (layer "F.Cu") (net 9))
 (segment (start 92.672 54.064) (end 93.434 54.064) (width 0.4) (layer "F.Cu") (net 9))
 (segment (start 93.434 54.064) (end 93.434 59.906) (width 0.4) (layer "F.Cu") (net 9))
 (segment (start 92.164 53.048) (end 92.164 53.556) (width 0.4) (layer "F.Cu") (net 9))
 (segment (start 92.418 53.556) (end 92.418 53.81) (width 0.4) (layer "F.Cu") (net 9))
 (segment (start 91.984999 53) (end 91.91 53.048) (width 0.4) (layer "F.Cu") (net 9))
 (segment (start 93.434 59.906) (end 93.5 60) (width 0.4) (layer "F.Cu") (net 9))
 (segment (start 92.418 53.81) (end 92.672 53.81) (width 0.4) (layer "F.Cu") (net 9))
 (segment (start 92.164 53.556) (end 92.418 53.556) (width 0.4) (layer "F.Cu") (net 9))
 (segment (start 93.434 53.556) (end 93.688 53.556) (width 0.4) (layer "B.Cu") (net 10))
 (segment (start 93.254999 53) (end 93.18 53.048) (width 0.4) (layer "B.Cu") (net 10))
 (segment (start 93.688 53.81) (end 93.942 53.81) (width 0.4) (layer "B.Cu") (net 10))
 (segment (start 100.545999 59.906) (end 100.5 60) (width 0.4) (layer "B.Cu") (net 10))
 (segment (start 93.434 53.048) (end 93.434 53.556) (width 0.4) (layer "B.Cu") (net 10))
 (segment (start 100.545999 54.064) (end 100.545999 59.906) (width 0.4) (layer "B.Cu") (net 10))
 (segment (start 93.688 53.556) (end 93.688 53.81) (width 0.4) (layer "B.Cu") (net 10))
 (segment (start 93.18 53.048) (end 93.434 53.048) (width 0.4) (layer "B.Cu") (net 10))
 (segment (start 93.942 53.81) (end 93.942 54.064) (width 0.4) (layer "B.Cu") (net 10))
 (segment (start 93.942 54.064) (end 100.545999 54.064) (width 0.4) (layer "B.Cu") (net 10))
 (segment (start 98.006 59.906) (end 98 60) (width 0.4) (layer "F.Cu") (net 11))
 (segment (start 94.704 53.556) (end 94.958 53.556) (width 0.4) (layer "F.Cu") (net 11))
 (segment (start 94.704 53.048) (end 94.704 53.556) (width 0.4) (layer "F.Cu") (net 11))
 (segment (start 95.212 54.064) (end 98.006 54.064) (width 0.4) (layer "F.Cu") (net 11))
 (segment (start 94.958 53.81) (end 95.212 53.81) (width 0.4) (layer "F.Cu") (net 11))
 (segment (start 94.524999 53) (end 94.45 53.048) (width 0.4) (layer "F.Cu") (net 11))
 (segment (start 98.006 54.064) (end 98.006 59.906) (width 0.4) (layer "F.Cu") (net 11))
 (segment (start 94.958 53.556) (end 94.958 53.81) (width 0.4) (layer "F.Cu") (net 11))
 (segment (start 95.212 53.81) (end 95.212 54.064) (width 0.4) (layer "F.Cu") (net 11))
 (segment (start 94.45 53.048) (end 94.704 53.048) (width 0.4) (layer "F.Cu") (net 11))
 (segment (start 96.228 52.032) (end 96.736 52.032) (width 0.4) (layer "F.Cu") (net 12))
 (segment (start 95.794999 53) (end 95.72 53.048) (width 0.4) (layer "F.Cu") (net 12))
 (segment (start 96.736 52.032) (end 96.736 51.778) (width 0.4) (layer "F.Cu") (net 12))
 (segment (start 103.086 59.906) (end 103.086 64.986) (width 0.4) (layer "F.Cu") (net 12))
 (segment (start 95.72 53.048) (end 95.974 53.048) (width 0.4) (layer "F.Cu") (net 12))
 (segment (start 96.228 52.286) (end 96.228 52.032) (width 0.4) (layer "F.Cu") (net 12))
 (segment (start 95.974 52.286) (end 96.228 52.286) (width 0.4) (layer "F.Cu") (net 12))
 (segment (start 95.974 53.048) (end 95.974 52.286) (width 0.4) (layer "F.Cu") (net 12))
 (segment (start 96.736 51.778) (end 105.118 51.778) (width 0.4) (layer "F.Cu") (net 12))
 (segment (start 105 60) (end 105.118 59.906) (width 0.4) (layer "F.Cu") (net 12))
 (segment (start 103.086 64.986) (end 103 65) (width 0.4) (layer "F.Cu") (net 12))
 (segment (start 105.118 59.906) (end 103.086 59.906) (width 0.4) (layer "F.Cu") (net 12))
 (segment (start 105.118 59.906) (end 105 60) (width 0.4) (layer "F.Cu") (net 12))
 (segment (start 105.118 51.778) (end 105.118 59.906) (width 0.4) (layer "F.Cu") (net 12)))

